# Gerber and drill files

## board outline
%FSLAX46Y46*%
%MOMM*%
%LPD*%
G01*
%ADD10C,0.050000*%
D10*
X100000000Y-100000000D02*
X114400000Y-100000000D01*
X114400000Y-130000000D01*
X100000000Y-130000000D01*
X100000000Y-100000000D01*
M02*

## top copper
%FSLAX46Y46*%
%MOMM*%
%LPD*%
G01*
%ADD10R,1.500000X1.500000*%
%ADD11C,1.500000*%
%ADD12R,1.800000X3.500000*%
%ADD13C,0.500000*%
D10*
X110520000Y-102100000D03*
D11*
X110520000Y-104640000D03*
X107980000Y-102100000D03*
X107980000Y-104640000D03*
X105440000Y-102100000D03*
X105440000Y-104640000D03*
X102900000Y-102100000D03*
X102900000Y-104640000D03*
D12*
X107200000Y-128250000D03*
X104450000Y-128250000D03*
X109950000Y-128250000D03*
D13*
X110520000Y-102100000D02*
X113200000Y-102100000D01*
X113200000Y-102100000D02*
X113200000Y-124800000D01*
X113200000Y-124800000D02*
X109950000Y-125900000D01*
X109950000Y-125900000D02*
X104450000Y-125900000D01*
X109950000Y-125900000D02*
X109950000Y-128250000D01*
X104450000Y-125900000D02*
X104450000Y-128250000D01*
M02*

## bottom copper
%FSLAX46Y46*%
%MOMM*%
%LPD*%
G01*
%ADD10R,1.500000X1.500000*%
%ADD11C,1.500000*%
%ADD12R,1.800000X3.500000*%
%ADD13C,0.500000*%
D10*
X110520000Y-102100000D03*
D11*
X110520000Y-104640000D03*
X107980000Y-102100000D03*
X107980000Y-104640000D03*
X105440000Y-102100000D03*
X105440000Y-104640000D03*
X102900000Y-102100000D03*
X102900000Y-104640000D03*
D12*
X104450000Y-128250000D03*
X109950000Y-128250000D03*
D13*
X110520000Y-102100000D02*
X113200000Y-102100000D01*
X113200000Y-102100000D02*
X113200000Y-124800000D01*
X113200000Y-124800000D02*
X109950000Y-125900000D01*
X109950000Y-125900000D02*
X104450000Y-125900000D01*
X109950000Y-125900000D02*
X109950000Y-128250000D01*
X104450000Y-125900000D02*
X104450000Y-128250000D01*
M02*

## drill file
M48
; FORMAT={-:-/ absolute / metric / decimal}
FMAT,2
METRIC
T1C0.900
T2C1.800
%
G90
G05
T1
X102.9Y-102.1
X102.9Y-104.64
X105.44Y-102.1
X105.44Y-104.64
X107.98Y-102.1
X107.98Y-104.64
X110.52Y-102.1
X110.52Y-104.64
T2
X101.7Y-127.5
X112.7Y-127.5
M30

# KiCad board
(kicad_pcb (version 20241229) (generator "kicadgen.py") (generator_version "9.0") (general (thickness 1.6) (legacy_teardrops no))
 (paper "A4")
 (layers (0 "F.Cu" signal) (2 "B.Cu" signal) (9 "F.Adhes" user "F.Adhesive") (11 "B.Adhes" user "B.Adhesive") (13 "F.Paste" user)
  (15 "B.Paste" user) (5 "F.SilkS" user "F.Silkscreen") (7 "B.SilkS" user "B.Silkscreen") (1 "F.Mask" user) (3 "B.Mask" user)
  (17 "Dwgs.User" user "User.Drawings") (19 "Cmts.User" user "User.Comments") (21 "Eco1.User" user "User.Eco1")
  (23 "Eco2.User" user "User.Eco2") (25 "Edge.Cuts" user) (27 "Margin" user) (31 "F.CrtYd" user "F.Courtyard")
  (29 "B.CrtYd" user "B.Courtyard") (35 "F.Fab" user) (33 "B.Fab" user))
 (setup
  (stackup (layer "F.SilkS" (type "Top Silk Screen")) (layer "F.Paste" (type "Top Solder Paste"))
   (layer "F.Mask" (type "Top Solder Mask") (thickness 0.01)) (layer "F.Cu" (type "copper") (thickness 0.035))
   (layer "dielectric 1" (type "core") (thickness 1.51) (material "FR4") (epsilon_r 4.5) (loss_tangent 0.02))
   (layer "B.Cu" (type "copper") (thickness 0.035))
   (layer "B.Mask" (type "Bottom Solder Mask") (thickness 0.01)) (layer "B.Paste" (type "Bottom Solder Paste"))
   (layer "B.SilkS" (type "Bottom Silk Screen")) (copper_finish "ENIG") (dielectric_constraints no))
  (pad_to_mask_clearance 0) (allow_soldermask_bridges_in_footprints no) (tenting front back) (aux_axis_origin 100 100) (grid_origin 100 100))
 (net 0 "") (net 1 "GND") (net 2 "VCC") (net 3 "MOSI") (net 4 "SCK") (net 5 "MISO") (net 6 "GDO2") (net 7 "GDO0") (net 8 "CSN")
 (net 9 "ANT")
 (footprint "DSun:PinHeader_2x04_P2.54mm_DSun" (layer "F.Cu") (at 110.52 102.1)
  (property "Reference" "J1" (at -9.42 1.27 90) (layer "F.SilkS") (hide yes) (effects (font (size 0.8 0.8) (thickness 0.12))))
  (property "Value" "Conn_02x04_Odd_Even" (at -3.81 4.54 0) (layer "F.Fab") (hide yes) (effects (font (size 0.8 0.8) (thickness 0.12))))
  (pad "1" thru_hole rect (at 0 0) (size 1.5 1.5) (drill 0.9) (layers "*.Cu" "*.Mask") (remove_unused_layers no) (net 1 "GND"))
  (pad "2" thru_hole circle (at 0 2.54) (size 1.5 1.5) (drill 0.9) (layers "*.Cu" "*.Mask") (remove_unused_layers no) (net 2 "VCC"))
  (pad "3" thru_hole circle (at -2.54 0) (size 1.5 1.5) (drill 0.9) (layers "*.Cu" "*.Mask") (remove_unused_layers no) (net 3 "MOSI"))
  (pad "4" thru_hole circle (at -2.54 2.54) (size 1.5 1.5) (drill 0.9) (layers "*.Cu" "*.Mask") (remove_unused_layers no) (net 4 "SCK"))
  (pad "5" thru_hole circle (at -5.08 0) (size 1.5 1.5) (drill 0.9) (layers "*.Cu" "*.Mask") (remove_unused_layers no) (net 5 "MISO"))
  (pad "6" thru_hole circle (at -5.08 2.54) (size 1.5 1.5) (drill 0.9) (layers "*.Cu" "*.Mask") (remove_unused_layers no) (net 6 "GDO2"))
  (pad "7" thru_hole circle (at -7.62 0) (size 1.5 1.5) (drill 0.9) (layers "*.Cu" "*.Mask") (remove_unused_layers no) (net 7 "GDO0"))
  (pad "8" thru_hole circle (at -7.62 2.54) (size 1.5 1.5) (drill 0.9) (layers "*.Cu" "*.Mask") (remove_unused_layers no) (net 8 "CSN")))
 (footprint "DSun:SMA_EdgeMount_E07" (layer "F.Cu") (at 107.2 130)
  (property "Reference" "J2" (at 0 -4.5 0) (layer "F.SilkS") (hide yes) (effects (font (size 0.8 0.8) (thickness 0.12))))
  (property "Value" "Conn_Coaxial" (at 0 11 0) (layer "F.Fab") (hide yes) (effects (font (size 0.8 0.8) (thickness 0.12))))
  (pad "1" smd rect (at 0 -1.75) (size 1.8 3.5) (layers "F.Cu" "F.Mask" "F.Paste") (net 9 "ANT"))
  (pad "2" smd rect (at -2.75 -1.75) (size 1.8 3.5) (layers "F.Cu" "F.Mask" "F.Paste") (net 1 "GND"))
  (pad "2" smd rect (at -2.75 -1.75) (size 1.8 3.5) (layers "B.Cu" "B.Mask" "B.Paste") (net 1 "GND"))
  (pad "2" smd rect (at 2.75 -1.75) (size 1.8 3.5) (layers "F.Cu" "F.Mask" "F.Paste") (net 1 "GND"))
  (pad "2" smd rect (at 2.75 -1.75) (size 1.8 3.5) (layers "B.Cu" "B.Mask" "B.Paste") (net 1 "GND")))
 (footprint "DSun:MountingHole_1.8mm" (layer "F.Cu") (at 101.7 127.5)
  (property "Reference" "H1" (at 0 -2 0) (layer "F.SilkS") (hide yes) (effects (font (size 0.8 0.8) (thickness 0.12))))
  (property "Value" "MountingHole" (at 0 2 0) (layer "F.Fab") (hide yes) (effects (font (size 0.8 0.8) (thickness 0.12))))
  (pad "1" np_thru_hole circle (at 0 0) (size 1.8 1.8) (drill 1.8) (layers "*.Cu" "*.Mask")))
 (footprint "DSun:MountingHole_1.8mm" (layer "F.Cu") (at 112.7 127.5)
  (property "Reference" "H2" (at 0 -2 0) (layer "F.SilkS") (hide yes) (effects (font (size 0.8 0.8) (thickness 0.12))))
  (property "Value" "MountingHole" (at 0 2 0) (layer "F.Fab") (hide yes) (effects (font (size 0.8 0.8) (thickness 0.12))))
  (pad "1" np_thru_hole circle (at 0 0) (size 1.8 1.8) (drill 1.8) (layers "*.Cu" "*.Mask")))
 (gr_rect (start 100 100) (end 114.4 130) (stroke (width 0.05) (type solid)) (fill no) (layer "Edge.Cuts"))
 (segment (start 110.52 102.1) (end 113.2 102.1) (width 0.5) (layer "F.Cu") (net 1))
 (segment (start 113.2 102.1) (end 113.2 124.8) (width 0.5) (layer "F.Cu") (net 1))
 (segment (start 113.2 124.8) (end 109.95 125.9) (width 0.5) (layer "F.Cu") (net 1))
 (segment (start 109.95 125.9) (end 104.45 125.9) (width 0.5) (layer "F.Cu") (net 1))
 (segment (start 109.95 125.9) (end 109.95 128.25) (width 0.5) (layer "F.Cu") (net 1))
 (segment (start 104.45 125.9) (end 104.45 128.25) (width 0.5) (layer "F.Cu") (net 1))
 (segment (start 110.52 102.1) (end 113.2 102.1) (width 0.5) (layer "B.Cu") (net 1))
 (segment (start 113.2 102.1) (end 113.2 124.8) (width 0.5) (layer "B.Cu") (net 1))
 (segment (start 113.2 124.8) (end 109.95 125.9) (width 0.5) (layer "B.Cu") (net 1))
 (segment (start 109.95 125.9) (end 104.45 125.9) (width 0.5) (layer "B.Cu") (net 1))
 (segment (start 109.95 125.9) (end 109.95 128.25) (width 0.5) (layer "B.Cu") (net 1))
 (segment (start 104.45 125.9) (end 104.45 128.25) (width 0.5) (layer "B.Cu") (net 1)))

